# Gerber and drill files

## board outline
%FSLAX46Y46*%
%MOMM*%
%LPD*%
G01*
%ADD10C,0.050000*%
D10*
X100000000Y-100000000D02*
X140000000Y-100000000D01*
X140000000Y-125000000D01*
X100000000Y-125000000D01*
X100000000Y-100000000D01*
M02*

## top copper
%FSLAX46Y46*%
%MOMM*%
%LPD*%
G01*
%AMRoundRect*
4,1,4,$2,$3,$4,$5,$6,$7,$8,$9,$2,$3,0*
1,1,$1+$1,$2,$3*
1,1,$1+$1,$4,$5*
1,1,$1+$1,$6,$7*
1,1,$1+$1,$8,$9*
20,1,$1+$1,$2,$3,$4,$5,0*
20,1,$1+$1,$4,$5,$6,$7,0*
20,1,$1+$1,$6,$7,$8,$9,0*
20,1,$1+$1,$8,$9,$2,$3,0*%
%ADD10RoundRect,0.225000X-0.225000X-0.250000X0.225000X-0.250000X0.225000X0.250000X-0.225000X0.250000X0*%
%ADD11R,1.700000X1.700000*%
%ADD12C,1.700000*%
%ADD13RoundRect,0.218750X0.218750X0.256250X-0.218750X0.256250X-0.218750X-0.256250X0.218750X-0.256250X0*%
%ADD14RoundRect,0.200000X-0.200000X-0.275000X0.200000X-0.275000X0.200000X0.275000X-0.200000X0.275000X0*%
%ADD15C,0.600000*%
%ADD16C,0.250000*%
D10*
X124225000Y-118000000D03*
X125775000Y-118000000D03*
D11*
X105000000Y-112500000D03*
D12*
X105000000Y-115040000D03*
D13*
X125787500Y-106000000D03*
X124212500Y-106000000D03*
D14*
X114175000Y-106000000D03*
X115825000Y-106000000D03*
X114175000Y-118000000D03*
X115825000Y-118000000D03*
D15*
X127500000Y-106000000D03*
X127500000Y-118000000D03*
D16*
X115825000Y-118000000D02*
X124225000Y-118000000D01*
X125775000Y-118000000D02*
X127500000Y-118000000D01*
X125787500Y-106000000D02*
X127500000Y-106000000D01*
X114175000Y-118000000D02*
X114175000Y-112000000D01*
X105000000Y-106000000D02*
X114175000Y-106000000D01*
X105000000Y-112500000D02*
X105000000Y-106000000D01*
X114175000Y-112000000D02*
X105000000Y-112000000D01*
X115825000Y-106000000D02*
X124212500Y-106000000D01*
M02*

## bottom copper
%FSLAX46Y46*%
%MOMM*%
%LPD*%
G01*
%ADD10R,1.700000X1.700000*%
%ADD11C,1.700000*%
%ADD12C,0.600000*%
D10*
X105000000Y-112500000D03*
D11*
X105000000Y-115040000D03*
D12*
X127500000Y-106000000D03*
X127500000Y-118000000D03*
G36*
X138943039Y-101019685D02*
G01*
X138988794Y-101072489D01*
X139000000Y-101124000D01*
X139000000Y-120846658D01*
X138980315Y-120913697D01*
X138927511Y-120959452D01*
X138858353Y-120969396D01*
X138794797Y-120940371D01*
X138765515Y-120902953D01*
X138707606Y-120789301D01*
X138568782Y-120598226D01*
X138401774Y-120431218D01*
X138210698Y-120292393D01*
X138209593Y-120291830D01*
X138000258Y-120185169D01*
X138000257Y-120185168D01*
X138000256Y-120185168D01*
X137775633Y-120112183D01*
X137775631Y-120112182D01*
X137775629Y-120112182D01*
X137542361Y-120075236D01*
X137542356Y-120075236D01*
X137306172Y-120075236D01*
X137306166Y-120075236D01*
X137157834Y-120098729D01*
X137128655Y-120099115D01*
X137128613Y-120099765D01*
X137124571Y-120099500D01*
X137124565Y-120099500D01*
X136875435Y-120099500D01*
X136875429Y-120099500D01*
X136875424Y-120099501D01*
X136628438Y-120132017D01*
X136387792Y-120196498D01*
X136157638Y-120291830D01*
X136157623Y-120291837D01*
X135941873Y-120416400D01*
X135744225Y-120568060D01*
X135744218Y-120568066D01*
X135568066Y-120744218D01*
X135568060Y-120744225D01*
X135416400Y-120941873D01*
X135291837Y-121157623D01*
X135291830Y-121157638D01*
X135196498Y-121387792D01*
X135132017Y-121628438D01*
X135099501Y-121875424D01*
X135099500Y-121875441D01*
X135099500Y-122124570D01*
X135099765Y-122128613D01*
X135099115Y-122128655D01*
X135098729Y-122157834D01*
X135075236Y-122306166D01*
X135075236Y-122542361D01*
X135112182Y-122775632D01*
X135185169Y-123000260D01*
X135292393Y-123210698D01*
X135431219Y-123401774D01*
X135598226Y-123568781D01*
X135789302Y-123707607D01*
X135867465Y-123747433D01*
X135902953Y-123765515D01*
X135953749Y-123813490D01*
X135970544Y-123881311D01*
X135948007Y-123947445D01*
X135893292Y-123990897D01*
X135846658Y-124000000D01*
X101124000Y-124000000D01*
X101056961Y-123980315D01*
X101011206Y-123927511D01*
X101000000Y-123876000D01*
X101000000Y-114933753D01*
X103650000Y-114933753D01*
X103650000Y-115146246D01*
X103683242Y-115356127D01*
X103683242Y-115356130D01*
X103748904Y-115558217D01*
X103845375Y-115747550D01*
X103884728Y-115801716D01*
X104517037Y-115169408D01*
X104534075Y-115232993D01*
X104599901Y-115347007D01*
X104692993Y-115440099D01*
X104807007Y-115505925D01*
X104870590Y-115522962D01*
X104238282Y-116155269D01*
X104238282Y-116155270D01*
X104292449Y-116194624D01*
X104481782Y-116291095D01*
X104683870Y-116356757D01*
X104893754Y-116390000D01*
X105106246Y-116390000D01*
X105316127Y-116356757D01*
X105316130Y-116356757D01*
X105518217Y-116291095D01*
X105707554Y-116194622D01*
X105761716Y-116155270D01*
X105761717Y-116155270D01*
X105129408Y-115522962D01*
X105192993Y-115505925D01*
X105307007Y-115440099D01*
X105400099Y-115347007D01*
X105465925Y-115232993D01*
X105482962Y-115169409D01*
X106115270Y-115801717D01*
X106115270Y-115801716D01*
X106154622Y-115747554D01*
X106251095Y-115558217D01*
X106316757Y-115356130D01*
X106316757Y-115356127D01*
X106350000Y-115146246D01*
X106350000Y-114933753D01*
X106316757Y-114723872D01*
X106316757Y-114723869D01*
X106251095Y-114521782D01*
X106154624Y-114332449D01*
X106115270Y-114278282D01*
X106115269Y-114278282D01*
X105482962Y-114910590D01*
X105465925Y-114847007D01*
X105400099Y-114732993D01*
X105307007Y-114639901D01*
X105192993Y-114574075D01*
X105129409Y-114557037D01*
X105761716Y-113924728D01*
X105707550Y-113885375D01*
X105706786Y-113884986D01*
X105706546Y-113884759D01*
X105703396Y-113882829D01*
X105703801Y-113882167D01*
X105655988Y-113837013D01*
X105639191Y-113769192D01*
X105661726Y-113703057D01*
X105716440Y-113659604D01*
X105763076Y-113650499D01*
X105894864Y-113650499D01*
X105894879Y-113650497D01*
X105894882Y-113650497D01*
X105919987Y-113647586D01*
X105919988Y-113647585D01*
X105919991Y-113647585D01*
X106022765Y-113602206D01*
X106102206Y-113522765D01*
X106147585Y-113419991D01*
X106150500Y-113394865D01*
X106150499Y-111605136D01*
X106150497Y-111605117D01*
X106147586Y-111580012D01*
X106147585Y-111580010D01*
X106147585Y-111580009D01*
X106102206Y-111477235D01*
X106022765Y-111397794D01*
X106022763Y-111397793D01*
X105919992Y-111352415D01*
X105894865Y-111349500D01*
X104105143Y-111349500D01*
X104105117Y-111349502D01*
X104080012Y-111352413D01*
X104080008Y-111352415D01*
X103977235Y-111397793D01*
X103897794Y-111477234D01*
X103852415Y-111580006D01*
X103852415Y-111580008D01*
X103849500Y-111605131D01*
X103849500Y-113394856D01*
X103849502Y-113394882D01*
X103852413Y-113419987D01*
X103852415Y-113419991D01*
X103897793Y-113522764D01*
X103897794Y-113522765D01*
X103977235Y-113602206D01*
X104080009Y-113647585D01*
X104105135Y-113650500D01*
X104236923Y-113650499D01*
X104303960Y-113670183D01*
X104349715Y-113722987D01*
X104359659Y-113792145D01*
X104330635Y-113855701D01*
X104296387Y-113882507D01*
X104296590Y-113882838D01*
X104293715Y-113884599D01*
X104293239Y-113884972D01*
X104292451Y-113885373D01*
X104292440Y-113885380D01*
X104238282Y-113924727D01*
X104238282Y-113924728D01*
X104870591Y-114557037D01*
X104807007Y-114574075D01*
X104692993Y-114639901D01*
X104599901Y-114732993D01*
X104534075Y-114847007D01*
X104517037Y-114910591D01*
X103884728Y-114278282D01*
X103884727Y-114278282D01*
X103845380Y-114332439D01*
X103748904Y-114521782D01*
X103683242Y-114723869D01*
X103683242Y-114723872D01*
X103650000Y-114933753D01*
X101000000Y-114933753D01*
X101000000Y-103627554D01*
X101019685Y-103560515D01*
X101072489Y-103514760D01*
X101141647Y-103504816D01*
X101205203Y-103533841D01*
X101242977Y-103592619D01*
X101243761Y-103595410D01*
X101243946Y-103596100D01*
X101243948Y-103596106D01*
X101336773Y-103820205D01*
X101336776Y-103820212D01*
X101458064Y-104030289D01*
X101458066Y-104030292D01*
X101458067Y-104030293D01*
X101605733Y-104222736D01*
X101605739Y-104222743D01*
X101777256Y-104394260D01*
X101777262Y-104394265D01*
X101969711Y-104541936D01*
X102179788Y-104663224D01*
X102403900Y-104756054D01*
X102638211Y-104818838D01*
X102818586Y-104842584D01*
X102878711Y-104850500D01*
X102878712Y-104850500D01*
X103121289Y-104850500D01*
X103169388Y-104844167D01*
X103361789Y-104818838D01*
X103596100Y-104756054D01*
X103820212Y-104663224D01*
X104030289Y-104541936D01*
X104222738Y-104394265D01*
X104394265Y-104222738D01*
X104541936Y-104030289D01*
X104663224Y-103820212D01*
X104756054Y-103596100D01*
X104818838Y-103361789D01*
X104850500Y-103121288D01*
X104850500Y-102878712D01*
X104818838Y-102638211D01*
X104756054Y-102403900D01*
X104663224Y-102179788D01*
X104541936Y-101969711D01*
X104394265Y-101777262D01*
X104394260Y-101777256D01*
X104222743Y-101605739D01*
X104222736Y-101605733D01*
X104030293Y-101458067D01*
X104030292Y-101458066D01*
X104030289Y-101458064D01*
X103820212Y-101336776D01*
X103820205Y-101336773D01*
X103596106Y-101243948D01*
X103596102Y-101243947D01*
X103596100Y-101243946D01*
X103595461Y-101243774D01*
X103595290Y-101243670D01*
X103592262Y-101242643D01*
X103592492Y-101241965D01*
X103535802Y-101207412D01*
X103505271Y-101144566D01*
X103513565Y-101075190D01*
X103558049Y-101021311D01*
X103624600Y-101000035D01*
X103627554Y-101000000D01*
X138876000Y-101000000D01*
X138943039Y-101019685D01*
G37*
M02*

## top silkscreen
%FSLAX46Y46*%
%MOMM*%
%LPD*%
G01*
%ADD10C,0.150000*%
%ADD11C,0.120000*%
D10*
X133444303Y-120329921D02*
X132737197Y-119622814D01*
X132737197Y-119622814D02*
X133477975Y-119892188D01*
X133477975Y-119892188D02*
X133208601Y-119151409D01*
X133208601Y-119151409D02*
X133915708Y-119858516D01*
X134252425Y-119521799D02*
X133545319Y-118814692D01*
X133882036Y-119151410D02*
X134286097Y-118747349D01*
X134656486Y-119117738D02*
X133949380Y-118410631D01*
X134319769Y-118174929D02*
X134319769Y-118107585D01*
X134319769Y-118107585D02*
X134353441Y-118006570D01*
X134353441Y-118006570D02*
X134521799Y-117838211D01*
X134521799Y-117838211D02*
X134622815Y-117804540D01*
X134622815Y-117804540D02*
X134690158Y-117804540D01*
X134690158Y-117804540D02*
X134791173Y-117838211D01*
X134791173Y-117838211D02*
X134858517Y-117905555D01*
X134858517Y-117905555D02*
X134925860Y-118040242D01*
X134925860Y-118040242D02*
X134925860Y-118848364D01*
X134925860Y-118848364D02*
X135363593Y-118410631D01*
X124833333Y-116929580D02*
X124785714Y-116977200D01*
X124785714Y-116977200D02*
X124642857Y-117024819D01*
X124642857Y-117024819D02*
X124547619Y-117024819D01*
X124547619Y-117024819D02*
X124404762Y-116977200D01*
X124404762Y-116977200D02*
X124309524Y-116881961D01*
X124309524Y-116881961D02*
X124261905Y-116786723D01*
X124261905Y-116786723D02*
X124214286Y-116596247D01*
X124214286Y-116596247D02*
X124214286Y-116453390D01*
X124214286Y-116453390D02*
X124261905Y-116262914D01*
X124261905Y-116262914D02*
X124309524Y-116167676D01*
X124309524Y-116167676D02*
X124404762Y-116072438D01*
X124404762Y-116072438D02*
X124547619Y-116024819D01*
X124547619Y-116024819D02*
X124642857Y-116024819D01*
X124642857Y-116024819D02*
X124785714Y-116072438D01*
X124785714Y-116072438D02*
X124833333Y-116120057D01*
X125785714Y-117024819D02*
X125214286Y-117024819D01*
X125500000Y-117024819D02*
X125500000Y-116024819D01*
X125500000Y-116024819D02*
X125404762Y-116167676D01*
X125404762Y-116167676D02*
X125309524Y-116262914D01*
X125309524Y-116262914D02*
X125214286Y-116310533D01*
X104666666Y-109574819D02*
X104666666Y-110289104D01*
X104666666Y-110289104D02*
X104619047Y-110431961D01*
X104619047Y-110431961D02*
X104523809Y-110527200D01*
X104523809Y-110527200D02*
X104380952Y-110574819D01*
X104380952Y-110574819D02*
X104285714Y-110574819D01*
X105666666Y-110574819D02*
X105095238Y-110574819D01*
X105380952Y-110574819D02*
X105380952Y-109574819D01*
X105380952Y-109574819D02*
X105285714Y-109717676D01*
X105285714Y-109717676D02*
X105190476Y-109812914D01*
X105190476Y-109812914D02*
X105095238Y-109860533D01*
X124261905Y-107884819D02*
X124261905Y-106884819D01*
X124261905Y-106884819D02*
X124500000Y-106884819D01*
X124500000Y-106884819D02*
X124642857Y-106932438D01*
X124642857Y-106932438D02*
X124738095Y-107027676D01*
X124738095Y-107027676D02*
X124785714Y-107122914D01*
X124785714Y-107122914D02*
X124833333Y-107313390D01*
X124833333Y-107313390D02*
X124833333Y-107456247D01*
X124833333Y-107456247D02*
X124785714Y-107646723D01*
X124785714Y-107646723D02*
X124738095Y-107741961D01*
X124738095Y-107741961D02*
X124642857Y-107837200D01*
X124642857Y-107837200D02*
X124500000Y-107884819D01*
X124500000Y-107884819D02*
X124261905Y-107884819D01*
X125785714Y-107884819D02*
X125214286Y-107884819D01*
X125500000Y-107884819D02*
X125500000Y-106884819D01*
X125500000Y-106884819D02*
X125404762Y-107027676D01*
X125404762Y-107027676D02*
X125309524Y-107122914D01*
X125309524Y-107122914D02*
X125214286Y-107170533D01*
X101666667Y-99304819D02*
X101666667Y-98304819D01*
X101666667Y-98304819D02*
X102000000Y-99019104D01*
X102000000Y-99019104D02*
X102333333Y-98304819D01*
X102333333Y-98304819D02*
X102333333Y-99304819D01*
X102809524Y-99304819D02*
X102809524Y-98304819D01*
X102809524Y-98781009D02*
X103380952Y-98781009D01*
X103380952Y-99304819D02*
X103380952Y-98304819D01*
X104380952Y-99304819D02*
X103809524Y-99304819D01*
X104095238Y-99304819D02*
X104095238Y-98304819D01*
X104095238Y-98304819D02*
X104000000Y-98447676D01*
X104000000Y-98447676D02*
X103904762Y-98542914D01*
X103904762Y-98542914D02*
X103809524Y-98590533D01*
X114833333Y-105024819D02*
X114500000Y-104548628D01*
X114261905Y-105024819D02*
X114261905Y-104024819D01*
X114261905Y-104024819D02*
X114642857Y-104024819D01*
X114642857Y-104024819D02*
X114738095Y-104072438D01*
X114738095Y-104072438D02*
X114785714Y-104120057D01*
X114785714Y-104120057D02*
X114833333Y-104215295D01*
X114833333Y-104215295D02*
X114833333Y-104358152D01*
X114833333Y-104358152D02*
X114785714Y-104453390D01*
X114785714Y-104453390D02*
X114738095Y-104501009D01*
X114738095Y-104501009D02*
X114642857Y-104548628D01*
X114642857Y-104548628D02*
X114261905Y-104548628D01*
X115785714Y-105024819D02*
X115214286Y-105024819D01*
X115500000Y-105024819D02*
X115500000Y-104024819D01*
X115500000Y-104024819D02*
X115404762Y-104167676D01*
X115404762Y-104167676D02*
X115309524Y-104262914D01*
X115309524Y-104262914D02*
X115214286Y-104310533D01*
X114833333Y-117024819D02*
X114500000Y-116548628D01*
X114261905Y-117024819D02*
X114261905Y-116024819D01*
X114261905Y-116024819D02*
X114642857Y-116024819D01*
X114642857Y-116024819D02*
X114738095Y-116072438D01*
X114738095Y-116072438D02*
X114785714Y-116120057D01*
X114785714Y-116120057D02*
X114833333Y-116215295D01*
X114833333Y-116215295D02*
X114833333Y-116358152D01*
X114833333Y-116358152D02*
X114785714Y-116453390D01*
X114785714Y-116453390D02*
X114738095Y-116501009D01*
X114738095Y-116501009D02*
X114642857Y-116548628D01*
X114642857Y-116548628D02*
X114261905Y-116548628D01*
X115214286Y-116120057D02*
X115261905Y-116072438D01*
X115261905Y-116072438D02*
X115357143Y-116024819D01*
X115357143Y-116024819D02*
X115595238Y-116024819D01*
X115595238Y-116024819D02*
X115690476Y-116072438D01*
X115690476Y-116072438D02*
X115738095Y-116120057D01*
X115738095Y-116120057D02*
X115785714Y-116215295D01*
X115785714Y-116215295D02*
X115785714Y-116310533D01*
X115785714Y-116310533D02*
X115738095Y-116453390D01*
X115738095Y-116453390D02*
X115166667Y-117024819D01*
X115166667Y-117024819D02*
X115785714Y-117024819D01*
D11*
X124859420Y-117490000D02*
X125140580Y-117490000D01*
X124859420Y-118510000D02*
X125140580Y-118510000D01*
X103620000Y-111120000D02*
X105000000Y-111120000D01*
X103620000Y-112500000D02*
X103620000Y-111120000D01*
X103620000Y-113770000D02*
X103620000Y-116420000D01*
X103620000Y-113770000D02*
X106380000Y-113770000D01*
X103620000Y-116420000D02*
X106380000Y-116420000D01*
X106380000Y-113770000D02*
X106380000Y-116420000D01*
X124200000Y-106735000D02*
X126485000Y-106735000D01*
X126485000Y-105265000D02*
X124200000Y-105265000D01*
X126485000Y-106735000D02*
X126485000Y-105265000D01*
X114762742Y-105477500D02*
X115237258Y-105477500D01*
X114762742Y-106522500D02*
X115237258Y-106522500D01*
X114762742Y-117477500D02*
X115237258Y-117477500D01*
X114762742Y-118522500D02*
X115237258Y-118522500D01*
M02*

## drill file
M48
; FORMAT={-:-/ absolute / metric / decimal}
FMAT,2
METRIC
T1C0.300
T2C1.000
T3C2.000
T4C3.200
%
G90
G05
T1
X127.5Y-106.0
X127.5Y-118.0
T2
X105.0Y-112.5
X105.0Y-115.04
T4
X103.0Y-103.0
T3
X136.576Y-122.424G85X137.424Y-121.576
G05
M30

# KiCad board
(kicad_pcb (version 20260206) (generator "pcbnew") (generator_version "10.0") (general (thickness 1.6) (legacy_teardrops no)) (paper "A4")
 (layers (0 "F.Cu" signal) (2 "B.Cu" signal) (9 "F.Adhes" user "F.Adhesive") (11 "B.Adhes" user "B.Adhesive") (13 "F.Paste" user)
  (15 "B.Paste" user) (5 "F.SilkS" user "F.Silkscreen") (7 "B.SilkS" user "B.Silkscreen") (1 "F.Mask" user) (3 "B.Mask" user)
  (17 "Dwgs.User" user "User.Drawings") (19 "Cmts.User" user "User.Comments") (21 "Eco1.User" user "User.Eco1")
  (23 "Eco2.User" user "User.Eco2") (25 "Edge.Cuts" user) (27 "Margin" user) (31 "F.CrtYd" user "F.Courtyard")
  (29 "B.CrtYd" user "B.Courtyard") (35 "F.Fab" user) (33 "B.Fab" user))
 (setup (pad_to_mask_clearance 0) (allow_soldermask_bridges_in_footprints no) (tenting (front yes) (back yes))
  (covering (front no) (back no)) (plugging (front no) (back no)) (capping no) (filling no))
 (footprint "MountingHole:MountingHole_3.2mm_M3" (layer "F.Cu") (at 137 122 45)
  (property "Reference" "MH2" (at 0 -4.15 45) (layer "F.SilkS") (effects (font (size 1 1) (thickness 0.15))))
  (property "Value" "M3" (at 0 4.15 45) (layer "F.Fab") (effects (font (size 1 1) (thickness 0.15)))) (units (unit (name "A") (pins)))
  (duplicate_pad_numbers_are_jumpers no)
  (pad "" np_thru_hole circle (at 0 0 45) (size 3.2 3.2) (drill oval 3.2 2) (layers "*.Cu" "*.Mask")))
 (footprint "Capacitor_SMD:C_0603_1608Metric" (layer "F.Cu") (at 125 118)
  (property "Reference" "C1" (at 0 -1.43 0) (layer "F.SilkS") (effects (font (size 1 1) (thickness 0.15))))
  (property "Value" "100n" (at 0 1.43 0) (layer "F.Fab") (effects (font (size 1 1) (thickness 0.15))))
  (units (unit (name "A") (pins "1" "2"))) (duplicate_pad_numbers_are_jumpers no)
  (fp_line (start -0.14058 -0.51) (end 0.14058 -0.51) (stroke (width 0.12) (type solid)) (layer "F.SilkS"))
  (fp_line (start -0.14058 0.51) (end 0.14058 0.51) (stroke (width 0.12) (type solid)) (layer "F.SilkS"))
  (pad "1" smd roundrect (at -0.775 0) (size 0.9 0.95) (layers "F.Cu" "F.Mask" "F.Paste") (roundrect_rratio 0.25) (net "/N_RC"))
  (pad "2" smd roundrect (at 0.775 0) (size 0.9 0.95) (layers "F.Cu" "F.Mask" "F.Paste") (roundrect_rratio 0.25) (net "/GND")))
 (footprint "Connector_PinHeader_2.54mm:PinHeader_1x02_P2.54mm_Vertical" (layer "F.Cu") (at 105 112.5)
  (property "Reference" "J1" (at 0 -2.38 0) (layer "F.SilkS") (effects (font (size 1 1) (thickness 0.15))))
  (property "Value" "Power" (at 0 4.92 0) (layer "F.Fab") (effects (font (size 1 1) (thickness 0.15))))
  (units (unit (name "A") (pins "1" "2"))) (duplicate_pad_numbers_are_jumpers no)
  (fp_line (start -1.38 -1.38) (end 0 -1.38) (stroke (width 0.12) (type solid)) (layer "F.SilkS"))
  (fp_line (start -1.38 0) (end -1.38 -1.38) (stroke (width 0.12) (type solid)) (layer "F.SilkS"))
  (fp_line (start -1.38 1.27) (end -1.38 3.92) (stroke (width 0.12) (type solid)) (layer "F.SilkS"))
  (fp_line (start -1.38 1.27) (end 1.38 1.27) (stroke (width 0.12) (type solid)) (layer "F.SilkS"))
  (fp_line (start -1.38 3.92) (end 1.38 3.92) (stroke (width 0.12) (type solid)) (layer "F.SilkS"))
  (fp_line (start 1.38 1.27) (end 1.38 3.92) (stroke (width 0.12) (type solid)) (layer "F.SilkS"))
  (pad "1" thru_hole rect (at 0 0) (size 1.7 1.7) (drill 1) (layers "*.Cu" "*.Mask") (remove_unused_layers no) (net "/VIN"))
  (pad "2" thru_hole circle (at 0 2.54) (size 1.7 1.7) (drill 1) (layers "*.Cu" "*.Mask") (remove_unused_layers no) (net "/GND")))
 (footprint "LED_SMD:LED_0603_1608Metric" (layer "F.Cu") (at 125 106 180)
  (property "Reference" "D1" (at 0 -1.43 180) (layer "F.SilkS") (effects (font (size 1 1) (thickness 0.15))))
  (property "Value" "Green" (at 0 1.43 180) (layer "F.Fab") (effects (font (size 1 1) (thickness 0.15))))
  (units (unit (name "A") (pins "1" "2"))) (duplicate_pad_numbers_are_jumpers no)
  (fp_line (start 0.8 -0.735) (end -1.485 -0.735) (stroke (width 0.12) (type solid)) (layer "F.SilkS"))
  (fp_line (start -1.485 0.735) (end 0.8 0.735) (stroke (width 0.12) (type solid)) (layer "F.SilkS"))
  (fp_line (start -1.485 -0.735) (end -1.485 0.735) (stroke (width 0.12) (type solid)) (layer "F.SilkS"))
  (pad "1" smd roundrect (at -0.7875 0 180) (size 0.875 0.95) (layers "F.Cu" "F.Mask" "F.Paste") (roundrect_rratio 0.25) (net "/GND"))
  (pad "2" smd roundrect (at 0.7875 0 180) (size 0.875 0.95) (layers "F.Cu" "F.Mask" "F.Paste") (roundrect_rratio 0.25) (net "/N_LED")))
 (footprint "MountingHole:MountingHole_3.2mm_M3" (layer "F.Cu") (at 103 103)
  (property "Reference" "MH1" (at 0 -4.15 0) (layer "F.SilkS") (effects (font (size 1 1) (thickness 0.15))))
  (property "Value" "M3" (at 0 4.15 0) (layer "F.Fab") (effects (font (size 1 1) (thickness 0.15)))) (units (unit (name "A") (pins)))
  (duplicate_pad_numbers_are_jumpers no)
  (pad "" np_thru_hole circle (at 0 0) (size 3.2 3.2) (drill 3.2) (layers "*.Cu" "*.Mask")))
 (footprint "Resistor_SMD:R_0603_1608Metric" (layer "F.Cu") (at 115 106)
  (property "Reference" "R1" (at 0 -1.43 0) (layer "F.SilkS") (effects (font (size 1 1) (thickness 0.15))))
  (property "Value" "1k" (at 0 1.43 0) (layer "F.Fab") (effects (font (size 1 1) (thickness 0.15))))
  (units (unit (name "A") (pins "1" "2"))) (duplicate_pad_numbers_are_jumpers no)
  (fp_line (start -0.237258 -0.5225) (end 0.237258 -0.5225) (stroke (width 0.12) (type solid)) (layer "F.SilkS"))
  (fp_line (start -0.237258 0.5225) (end 0.237258 0.5225) (stroke (width 0.12) (type solid)) (layer "F.SilkS"))
  (pad "1" smd roundrect (at -0.825 0) (size 0.8 0.95) (layers "F.Cu" "F.Mask" "F.Paste") (roundrect_rratio 0.25) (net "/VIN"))
  (pad "2" smd roundrect (at 0.825 0) (size 0.8 0.95) (layers "F.Cu" "F.Mask" "F.Paste") (roundrect_rratio 0.25) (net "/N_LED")))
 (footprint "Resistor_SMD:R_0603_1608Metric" (layer "F.Cu") (at 115 118)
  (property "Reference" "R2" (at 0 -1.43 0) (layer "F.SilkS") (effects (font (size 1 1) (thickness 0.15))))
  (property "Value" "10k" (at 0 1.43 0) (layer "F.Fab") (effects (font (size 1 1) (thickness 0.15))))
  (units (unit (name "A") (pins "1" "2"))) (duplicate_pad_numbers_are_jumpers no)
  (fp_line (start -0.237258 -0.5225) (end 0.237258 -0.5225) (stroke (width 0.12) (type solid)) (layer "F.SilkS"))
  (fp_line (start -0.237258 0.5225) (end 0.237258 0.5225) (stroke (width 0.12) (type solid)) (layer "F.SilkS"))
  (pad "1" smd roundrect (at -0.825 0) (size 0.8 0.95) (layers "F.Cu" "F.Mask" "F.Paste") (roundrect_rratio 0.25) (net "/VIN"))
  (pad "2" smd roundrect (at 0.825 0) (size 0.8 0.95) (layers "F.Cu" "F.Mask" "F.Paste") (roundrect_rratio 0.25) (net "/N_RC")))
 (gr_rect (start 100 100) (end 140 125) (stroke (width 0.05) (type default)) (fill no) (layer "Edge.Cuts"))
 (segment (start 115.825 118) (end 124.225 118) (width 0.25) (layer "F.Cu") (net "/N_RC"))
 (segment (start 125.775 118) (end 127.5 118) (width 0.25) (layer "F.Cu") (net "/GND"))
 (segment (start 125.7875 106) (end 127.5 106) (width 0.25) (layer "F.Cu") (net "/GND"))
 (via (at 127.5 106) (size 0.6) (drill 0.3) (layers "F.Cu" "B.Cu") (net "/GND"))
 (via (at 127.5 118) (size 0.6) (drill 0.3) (layers "F.Cu" "B.Cu") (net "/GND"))
 (segment (start 114.175 118) (end 114.175 112) (width 0.25) (layer "F.Cu") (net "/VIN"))
 (segment (start 105 106) (end 114.175 106) (width 0.25) (layer "F.Cu") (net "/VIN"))
 (segment (start 105 112.5) (end 105 106) (width 0.25) (layer "F.Cu") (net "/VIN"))
 (segment (start 114.175 112) (end 105 112) (width 0.25) (layer "F.Cu") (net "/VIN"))
 (segment (start 115.825 106) (end 124.2125 106) (width 0.25) (layer "F.Cu") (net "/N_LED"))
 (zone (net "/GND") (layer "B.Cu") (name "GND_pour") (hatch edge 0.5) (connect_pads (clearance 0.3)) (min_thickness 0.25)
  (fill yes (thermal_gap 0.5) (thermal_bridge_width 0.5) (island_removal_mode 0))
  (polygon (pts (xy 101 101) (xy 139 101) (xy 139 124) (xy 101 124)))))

